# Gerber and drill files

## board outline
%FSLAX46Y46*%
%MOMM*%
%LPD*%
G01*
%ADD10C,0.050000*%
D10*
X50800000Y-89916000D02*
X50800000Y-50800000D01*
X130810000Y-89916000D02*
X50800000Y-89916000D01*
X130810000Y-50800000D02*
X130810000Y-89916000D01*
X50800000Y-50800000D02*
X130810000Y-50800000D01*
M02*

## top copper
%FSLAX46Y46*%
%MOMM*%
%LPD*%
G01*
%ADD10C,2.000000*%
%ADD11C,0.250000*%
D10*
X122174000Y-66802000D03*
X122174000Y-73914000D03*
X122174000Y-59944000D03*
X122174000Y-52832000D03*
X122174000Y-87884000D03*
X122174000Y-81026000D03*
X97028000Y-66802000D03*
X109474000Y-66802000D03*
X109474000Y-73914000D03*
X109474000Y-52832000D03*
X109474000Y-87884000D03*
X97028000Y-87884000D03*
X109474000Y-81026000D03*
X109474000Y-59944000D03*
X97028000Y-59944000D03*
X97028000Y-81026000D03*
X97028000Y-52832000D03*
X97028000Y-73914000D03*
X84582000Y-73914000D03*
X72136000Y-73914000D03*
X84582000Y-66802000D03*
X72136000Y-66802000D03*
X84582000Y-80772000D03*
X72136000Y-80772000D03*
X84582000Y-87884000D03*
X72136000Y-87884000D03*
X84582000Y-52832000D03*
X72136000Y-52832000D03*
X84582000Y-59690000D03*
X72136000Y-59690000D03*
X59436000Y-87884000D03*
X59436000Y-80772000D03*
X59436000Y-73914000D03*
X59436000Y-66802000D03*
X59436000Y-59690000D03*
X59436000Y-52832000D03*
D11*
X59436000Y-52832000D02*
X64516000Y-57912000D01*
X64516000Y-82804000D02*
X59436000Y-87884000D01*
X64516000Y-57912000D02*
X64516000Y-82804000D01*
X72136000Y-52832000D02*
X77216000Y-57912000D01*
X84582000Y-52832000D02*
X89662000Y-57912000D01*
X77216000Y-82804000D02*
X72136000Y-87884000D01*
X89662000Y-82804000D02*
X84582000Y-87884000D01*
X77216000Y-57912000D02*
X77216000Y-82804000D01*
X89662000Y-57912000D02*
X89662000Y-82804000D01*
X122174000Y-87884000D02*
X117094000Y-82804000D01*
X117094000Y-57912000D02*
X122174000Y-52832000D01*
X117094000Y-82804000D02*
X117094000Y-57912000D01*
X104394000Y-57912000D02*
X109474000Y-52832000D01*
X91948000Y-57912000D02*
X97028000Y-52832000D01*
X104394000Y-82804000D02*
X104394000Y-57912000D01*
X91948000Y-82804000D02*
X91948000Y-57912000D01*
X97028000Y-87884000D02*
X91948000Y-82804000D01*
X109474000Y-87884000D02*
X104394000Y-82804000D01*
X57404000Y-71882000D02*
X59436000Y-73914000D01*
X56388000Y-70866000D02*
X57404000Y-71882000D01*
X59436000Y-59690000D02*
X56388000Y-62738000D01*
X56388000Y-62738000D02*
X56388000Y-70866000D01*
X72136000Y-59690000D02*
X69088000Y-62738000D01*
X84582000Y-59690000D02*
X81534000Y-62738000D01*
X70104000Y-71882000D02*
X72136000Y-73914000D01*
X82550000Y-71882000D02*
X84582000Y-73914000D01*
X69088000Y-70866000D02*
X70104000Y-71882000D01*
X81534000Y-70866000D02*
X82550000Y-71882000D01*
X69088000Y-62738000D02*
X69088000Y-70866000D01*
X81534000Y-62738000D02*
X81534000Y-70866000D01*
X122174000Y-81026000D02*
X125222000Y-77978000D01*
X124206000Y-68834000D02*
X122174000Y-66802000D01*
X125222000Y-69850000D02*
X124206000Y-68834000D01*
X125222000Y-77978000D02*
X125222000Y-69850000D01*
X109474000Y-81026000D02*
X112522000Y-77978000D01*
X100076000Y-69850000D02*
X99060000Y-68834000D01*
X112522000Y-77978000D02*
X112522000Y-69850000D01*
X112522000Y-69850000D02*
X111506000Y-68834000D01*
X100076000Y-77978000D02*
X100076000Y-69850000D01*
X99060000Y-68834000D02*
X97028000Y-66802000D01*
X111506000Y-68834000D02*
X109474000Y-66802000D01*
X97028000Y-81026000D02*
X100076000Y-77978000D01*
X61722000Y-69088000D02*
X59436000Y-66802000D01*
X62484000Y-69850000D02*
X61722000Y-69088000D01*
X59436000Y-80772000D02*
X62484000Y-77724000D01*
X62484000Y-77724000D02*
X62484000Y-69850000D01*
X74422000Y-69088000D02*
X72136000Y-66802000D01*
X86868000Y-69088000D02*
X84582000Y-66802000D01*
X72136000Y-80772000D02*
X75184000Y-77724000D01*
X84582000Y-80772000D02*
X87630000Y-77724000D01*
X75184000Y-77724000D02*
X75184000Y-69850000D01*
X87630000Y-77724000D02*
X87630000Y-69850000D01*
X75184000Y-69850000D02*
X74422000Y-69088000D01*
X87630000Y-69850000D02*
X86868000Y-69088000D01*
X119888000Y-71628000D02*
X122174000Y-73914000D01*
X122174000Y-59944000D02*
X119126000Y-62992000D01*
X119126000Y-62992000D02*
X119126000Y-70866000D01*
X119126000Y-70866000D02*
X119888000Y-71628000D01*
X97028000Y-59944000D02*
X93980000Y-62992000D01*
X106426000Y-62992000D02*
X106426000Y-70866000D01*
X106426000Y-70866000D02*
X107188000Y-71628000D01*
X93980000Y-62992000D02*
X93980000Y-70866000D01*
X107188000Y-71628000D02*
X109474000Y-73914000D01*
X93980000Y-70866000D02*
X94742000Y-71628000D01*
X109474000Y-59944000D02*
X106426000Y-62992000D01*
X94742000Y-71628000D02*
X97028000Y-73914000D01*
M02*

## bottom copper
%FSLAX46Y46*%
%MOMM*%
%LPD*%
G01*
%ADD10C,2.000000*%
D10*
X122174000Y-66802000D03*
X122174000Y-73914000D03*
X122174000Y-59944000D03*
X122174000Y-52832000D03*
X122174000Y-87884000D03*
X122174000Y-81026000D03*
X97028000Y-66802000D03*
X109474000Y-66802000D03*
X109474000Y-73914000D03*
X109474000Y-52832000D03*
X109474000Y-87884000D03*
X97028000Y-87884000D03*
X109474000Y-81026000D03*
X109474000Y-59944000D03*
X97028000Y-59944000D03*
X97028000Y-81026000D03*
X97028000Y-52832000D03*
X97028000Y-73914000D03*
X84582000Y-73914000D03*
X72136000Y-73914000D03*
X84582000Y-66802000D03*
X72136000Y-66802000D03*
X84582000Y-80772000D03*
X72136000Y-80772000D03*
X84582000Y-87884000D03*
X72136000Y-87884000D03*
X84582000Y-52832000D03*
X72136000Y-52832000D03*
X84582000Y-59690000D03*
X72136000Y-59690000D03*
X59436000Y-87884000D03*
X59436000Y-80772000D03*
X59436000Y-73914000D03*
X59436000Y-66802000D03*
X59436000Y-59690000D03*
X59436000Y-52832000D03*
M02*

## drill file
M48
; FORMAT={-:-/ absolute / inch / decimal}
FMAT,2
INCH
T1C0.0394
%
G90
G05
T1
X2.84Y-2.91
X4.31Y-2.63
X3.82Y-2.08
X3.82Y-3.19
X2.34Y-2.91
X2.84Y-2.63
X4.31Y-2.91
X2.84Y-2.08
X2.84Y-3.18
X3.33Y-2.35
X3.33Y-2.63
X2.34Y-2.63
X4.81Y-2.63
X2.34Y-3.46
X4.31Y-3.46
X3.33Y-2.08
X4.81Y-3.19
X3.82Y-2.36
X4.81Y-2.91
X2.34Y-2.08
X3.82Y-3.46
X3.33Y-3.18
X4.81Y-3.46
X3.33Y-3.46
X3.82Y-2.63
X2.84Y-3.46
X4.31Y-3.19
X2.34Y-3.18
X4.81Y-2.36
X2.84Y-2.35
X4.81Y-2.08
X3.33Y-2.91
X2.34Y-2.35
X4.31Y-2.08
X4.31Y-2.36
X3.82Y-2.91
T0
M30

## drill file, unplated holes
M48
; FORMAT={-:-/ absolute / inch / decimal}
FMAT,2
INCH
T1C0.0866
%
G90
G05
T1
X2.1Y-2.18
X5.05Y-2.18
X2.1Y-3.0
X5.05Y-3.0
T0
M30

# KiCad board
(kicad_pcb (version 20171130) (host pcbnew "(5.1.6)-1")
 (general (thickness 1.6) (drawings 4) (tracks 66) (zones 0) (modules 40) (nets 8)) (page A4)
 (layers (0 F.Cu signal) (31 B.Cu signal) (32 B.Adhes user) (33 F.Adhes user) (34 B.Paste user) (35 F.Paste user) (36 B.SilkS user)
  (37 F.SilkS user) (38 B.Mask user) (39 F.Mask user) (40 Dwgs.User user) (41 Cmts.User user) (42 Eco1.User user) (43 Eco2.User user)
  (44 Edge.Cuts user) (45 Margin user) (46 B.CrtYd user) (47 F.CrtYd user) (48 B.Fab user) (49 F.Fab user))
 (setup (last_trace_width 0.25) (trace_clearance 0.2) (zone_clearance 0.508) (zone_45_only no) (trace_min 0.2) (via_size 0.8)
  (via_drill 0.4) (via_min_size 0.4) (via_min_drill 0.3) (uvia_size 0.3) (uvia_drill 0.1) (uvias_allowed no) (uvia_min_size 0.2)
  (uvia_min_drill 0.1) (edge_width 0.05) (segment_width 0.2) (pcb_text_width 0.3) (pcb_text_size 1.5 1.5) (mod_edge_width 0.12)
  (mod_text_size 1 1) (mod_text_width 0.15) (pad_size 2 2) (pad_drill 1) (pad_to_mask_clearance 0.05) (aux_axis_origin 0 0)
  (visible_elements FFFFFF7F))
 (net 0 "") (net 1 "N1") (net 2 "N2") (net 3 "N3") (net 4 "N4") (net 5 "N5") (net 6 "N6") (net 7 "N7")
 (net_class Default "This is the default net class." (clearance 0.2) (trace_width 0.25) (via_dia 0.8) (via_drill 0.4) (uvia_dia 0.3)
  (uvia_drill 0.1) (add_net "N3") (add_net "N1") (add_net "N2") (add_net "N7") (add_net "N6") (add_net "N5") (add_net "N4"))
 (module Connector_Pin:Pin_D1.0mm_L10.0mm (layer F.Cu) (at 122.174 66.802 180)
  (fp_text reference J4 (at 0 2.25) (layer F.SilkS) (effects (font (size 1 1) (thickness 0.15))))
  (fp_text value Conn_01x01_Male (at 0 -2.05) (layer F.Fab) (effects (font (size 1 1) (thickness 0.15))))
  (pad 1 thru_hole circle (at 0 0 180) (size 2 2) (drill 1) (layers *.Cu *.Mask) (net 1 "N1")))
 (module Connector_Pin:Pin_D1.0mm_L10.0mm (layer F.Cu) (at 122.174 73.914 180)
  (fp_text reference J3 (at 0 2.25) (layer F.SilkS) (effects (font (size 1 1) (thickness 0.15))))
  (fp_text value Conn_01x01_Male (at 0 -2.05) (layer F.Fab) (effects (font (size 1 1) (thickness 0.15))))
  (pad 1 thru_hole circle (at 0 0 180) (size 2 2) (drill 1) (layers *.Cu *.Mask) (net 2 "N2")))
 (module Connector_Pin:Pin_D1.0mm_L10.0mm (layer F.Cu) (at 122.174 59.944 180)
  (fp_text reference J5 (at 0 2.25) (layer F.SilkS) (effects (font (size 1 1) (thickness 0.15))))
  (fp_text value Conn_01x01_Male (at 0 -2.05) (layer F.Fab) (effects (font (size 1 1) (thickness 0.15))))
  (pad 1 thru_hole circle (at 0 0 180) (size 2 2) (drill 1) (layers *.Cu *.Mask) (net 2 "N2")))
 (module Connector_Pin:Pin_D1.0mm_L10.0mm (layer F.Cu) (at 122.174 52.832 180)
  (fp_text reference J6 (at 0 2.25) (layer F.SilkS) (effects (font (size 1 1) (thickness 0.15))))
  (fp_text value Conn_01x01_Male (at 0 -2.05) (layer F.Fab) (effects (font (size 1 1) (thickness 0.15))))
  (pad 1 thru_hole circle (at 0 0 180) (size 2 2) (drill 1) (layers *.Cu *.Mask) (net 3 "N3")))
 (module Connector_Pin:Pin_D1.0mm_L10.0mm (layer F.Cu) (at 122.174 87.884 180)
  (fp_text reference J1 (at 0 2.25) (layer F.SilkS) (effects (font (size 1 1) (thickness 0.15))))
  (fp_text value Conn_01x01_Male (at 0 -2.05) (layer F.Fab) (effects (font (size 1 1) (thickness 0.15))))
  (pad 1 thru_hole circle (at 0 0 180) (size 2 2) (drill 1) (layers *.Cu *.Mask) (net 3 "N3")))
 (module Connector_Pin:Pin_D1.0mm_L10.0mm (layer F.Cu) (at 122.174 81.026 180)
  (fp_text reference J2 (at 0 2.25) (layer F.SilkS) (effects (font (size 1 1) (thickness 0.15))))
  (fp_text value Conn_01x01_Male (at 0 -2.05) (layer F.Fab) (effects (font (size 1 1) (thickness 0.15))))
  (pad 1 thru_hole circle (at 0 0 180) (size 2 2) (drill 1) (layers *.Cu *.Mask) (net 1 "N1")))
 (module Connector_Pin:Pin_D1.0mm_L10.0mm (layer F.Cu) (at 97.028 66.802 180)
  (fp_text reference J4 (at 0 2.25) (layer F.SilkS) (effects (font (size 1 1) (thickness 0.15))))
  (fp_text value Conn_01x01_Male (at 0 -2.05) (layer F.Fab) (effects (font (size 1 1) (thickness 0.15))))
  (pad 1 thru_hole circle (at 0 0 180) (size 2 2) (drill 1) (layers *.Cu *.Mask) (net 1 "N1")))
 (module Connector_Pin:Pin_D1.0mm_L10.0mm (layer F.Cu) (at 109.474 66.802 180)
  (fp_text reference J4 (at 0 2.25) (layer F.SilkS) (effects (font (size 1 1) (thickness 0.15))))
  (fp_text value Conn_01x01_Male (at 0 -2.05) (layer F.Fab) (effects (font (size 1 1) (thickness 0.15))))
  (pad 1 thru_hole circle (at 0 0 180) (size 2 2) (drill 1) (layers *.Cu *.Mask) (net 1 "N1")))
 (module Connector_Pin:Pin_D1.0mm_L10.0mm (layer F.Cu) (at 109.474 73.914 180)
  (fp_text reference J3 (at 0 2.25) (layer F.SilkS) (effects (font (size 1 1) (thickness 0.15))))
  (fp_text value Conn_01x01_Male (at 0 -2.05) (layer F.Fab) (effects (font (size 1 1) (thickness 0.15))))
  (pad 1 thru_hole circle (at 0 0 180) (size 2 2) (drill 1) (layers *.Cu *.Mask) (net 2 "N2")))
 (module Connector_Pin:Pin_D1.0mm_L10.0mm (layer F.Cu) (at 109.474 52.832 180)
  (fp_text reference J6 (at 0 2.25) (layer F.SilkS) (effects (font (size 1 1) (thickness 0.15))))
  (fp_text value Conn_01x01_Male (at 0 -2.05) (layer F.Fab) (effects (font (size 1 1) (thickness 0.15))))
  (pad 1 thru_hole circle (at 0 0 180) (size 2 2) (drill 1) (layers *.Cu *.Mask) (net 3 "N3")))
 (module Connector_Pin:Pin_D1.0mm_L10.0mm (layer F.Cu) (at 109.474 87.884 180)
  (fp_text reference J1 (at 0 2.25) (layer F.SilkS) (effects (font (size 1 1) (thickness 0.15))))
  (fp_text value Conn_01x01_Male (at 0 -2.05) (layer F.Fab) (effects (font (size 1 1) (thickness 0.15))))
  (pad 1 thru_hole circle (at 0 0 180) (size 2 2) (drill 1) (layers *.Cu *.Mask) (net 3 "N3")))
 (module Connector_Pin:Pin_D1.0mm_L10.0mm (layer F.Cu) (at 97.028 87.884 180)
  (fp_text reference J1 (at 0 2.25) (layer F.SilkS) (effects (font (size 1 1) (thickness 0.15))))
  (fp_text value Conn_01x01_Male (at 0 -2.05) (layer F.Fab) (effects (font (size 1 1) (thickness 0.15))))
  (pad 1 thru_hole circle (at 0 0 180) (size 2 2) (drill 1) (layers *.Cu *.Mask) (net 3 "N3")))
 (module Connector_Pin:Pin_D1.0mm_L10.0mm (layer F.Cu) (at 109.474 81.026 180)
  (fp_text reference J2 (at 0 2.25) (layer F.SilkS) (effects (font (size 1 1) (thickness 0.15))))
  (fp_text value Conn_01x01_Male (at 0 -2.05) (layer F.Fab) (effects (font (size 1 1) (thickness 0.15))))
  (pad 1 thru_hole circle (at 0 0 180) (size 2 2) (drill 1) (layers *.Cu *.Mask) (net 1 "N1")))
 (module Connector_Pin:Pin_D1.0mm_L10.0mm (layer F.Cu) (at 109.474 59.944 180)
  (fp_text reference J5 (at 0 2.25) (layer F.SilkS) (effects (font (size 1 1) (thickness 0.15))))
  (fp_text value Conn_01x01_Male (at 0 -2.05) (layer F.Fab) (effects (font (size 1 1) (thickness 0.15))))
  (pad 1 thru_hole circle (at 0 0 180) (size 2 2) (drill 1) (layers *.Cu *.Mask) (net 2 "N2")))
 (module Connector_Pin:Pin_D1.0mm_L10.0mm (layer F.Cu) (at 97.028 59.944 180)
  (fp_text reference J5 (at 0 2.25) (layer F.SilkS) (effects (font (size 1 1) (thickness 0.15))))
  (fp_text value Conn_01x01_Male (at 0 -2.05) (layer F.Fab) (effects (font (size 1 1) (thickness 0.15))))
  (pad 1 thru_hole circle (at 0 0 180) (size 2 2) (drill 1) (layers *.Cu *.Mask) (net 2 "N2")))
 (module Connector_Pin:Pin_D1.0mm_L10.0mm (layer F.Cu) (at 97.028 81.026 180)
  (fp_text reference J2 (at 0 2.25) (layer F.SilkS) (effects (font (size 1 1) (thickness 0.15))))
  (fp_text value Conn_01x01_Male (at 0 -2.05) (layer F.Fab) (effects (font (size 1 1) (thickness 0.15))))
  (pad 1 thru_hole circle (at 0 0 180) (size 2 2) (drill 1) (layers *.Cu *.Mask) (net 1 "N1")))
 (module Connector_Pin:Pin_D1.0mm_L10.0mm (layer F.Cu) (at 97.028 52.832 180)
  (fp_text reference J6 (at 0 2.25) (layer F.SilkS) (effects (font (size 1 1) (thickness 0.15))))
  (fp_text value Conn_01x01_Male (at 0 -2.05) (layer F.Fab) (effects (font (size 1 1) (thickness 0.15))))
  (pad 1 thru_hole circle (at 0 0 180) (size 2 2) (drill 1) (layers *.Cu *.Mask) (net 3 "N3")))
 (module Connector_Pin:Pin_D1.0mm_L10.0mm (layer F.Cu) (at 97.028 73.914 180)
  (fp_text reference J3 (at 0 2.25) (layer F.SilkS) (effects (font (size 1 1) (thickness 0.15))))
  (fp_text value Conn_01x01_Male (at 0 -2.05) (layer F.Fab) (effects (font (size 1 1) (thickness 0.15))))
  (pad 1 thru_hole circle (at 0 0 180) (size 2 2) (drill 1) (layers *.Cu *.Mask) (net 2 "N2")))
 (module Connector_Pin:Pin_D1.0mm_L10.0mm (layer F.Cu) (at 84.582 73.914)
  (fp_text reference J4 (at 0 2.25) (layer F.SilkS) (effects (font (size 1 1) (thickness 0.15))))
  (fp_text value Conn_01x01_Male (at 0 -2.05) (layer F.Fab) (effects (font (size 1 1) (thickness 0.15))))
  (pad 1 thru_hole circle (at 0 0) (size 2 2) (drill 1) (layers *.Cu *.Mask) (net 1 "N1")))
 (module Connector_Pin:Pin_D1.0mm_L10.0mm (layer F.Cu) (at 72.136 73.914)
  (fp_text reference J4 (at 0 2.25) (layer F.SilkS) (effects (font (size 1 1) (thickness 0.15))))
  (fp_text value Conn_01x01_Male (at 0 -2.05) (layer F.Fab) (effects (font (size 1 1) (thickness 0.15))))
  (pad 1 thru_hole circle (at 0 0) (size 2 2) (drill 1) (layers *.Cu *.Mask) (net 1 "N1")))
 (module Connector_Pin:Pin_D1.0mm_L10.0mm (layer F.Cu) (at 84.582 66.802)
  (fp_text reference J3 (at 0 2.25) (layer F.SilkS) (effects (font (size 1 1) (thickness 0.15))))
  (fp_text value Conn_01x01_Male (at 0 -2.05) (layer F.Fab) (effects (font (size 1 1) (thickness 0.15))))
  (pad 1 thru_hole circle (at 0 0) (size 2 2) (drill 1) (layers *.Cu *.Mask) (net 2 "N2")))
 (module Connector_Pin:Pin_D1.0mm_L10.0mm (layer F.Cu) (at 72.136 66.802)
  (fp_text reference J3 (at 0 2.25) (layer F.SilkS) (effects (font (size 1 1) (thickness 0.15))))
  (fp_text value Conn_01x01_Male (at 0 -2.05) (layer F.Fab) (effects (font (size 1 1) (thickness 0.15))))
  (pad 1 thru_hole circle (at 0 0) (size 2 2) (drill 1) (layers *.Cu *.Mask) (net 2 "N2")))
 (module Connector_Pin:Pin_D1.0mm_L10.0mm (layer F.Cu) (at 84.582 80.772)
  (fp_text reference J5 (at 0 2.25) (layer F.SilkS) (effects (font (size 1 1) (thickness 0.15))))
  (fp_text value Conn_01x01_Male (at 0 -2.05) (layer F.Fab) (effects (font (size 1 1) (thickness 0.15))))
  (pad 1 thru_hole circle (at 0 0) (size 2 2) (drill 1) (layers *.Cu *.Mask) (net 2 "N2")))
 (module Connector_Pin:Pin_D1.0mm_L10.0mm (layer F.Cu) (at 72.136 80.772)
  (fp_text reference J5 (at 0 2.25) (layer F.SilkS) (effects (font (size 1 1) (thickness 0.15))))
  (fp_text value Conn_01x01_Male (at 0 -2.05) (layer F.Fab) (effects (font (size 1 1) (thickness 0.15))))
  (pad 1 thru_hole circle (at 0 0) (size 2 2) (drill 1) (layers *.Cu *.Mask) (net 2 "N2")))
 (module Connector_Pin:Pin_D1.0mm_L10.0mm (layer F.Cu) (at 84.582 87.884)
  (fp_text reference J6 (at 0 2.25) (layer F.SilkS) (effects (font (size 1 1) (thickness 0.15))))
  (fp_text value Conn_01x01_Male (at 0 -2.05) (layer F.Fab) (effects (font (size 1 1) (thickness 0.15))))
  (pad 1 thru_hole circle (at 0 0) (size 2 2) (drill 1) (layers *.Cu *.Mask) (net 3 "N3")))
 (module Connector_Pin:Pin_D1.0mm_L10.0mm (layer F.Cu) (at 72.136 87.884)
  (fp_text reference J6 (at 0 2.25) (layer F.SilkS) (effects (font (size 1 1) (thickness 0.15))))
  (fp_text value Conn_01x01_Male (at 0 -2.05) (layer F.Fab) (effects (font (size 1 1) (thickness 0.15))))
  (pad 1 thru_hole circle (at 0 0) (size 2 2) (drill 1) (layers *.Cu *.Mask) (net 3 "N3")))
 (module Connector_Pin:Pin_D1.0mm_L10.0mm (layer F.Cu) (at 84.582 52.832)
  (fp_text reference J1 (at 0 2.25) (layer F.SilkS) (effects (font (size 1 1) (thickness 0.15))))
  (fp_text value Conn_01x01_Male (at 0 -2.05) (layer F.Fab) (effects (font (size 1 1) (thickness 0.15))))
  (pad 1 thru_hole circle (at 0 0) (size 2 2) (drill 1) (layers *.Cu *.Mask) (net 3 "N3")))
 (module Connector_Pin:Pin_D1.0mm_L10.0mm (layer F.Cu) (at 72.136 52.832)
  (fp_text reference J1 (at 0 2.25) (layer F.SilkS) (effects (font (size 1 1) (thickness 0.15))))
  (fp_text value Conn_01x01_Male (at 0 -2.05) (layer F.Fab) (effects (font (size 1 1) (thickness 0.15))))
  (pad 1 thru_hole circle (at 0 0) (size 2 2) (drill 1) (layers *.Cu *.Mask) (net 3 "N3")))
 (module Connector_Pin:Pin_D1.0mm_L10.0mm (layer F.Cu) (at 84.582 59.69)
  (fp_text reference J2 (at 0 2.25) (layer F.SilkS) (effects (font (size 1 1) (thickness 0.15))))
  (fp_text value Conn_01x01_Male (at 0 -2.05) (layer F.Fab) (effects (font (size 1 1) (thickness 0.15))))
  (pad 1 thru_hole circle (at 0 0) (size 2 2) (drill 1) (layers *.Cu *.Mask) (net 1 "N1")))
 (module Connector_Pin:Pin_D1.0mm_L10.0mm (layer F.Cu) (at 72.136 59.69)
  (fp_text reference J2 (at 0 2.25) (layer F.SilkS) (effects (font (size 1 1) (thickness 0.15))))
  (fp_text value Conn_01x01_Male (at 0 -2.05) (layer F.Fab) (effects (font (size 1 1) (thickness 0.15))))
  (pad 1 thru_hole circle (at 0 0) (size 2 2) (drill 1) (layers *.Cu *.Mask) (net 1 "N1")))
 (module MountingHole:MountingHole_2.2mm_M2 (layer F.Cu) (at 53.34 76.2)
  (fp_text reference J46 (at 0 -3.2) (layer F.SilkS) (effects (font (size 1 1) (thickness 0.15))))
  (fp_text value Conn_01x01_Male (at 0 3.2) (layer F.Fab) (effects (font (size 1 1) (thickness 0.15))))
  (pad 1 np_thru_hole circle (at 0 0) (size 2.2 2.2) (drill 2.2) (layers *.Cu *.Mask) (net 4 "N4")))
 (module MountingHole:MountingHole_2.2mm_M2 (layer F.Cu) (at 128.27 76.2)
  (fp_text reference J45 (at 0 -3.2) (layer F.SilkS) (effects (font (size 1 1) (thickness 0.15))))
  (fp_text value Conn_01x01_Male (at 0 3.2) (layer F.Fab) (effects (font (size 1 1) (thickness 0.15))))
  (pad 1 np_thru_hole circle (at 0 0) (size 2.2 2.2) (drill 2.2) (layers *.Cu *.Mask) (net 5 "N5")))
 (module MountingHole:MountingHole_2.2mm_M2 (layer F.Cu) (at 128.27 55.372)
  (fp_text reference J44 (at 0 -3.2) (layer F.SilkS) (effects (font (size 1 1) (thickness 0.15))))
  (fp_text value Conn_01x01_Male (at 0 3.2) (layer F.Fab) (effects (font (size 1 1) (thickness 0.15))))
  (pad 1 np_thru_hole circle (at 0 0) (size 2.2 2.2) (drill 2.2) (layers *.Cu *.Mask) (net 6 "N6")))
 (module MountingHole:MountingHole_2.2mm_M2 (layer F.Cu) (at 53.34 55.372)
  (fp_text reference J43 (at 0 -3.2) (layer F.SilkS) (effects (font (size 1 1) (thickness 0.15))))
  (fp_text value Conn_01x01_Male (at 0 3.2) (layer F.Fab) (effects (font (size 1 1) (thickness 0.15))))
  (pad 1 np_thru_hole circle (at 0 0) (size 2.2 2.2) (drill 2.2) (layers *.Cu *.Mask) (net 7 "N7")))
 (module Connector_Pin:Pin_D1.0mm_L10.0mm (layer F.Cu) (at 59.436 87.884)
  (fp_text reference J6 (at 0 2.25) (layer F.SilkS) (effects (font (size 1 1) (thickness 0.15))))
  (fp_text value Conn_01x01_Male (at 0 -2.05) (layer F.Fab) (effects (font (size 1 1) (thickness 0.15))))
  (pad 1 thru_hole circle (at 0 0) (size 2 2) (drill 1) (layers *.Cu *.Mask) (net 3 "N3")))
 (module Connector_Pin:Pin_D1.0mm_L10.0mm (layer F.Cu) (at 59.436 80.772)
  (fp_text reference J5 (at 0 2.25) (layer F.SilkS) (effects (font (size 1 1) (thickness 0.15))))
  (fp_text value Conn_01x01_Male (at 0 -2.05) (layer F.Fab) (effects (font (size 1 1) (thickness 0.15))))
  (pad 1 thru_hole circle (at 0 0) (size 2 2) (drill 1) (layers *.Cu *.Mask) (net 2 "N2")))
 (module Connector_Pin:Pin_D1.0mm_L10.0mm (layer F.Cu) (at 59.436 73.914)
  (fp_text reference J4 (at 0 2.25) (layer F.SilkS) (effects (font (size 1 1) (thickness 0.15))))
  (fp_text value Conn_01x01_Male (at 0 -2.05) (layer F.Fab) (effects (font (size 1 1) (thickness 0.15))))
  (pad 1 thru_hole circle (at 0 0) (size 2 2) (drill 1) (layers *.Cu *.Mask) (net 1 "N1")))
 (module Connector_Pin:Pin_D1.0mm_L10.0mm (layer F.Cu) (at 59.436 66.802)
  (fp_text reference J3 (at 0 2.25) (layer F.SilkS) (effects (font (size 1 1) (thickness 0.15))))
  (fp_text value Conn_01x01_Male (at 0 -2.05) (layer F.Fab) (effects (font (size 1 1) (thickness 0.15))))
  (pad 1 thru_hole circle (at 0 0) (size 2 2) (drill 1) (layers *.Cu *.Mask) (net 2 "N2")))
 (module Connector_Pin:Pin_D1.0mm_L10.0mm (layer F.Cu) (at 59.436 59.69)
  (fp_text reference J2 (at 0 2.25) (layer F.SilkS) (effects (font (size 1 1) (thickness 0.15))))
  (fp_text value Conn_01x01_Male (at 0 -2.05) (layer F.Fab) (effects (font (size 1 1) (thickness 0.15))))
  (pad 1 thru_hole circle (at 0 0) (size 2 2) (drill 1) (layers *.Cu *.Mask) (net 1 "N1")))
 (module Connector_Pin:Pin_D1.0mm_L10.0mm (layer F.Cu) (at 59.436 52.832)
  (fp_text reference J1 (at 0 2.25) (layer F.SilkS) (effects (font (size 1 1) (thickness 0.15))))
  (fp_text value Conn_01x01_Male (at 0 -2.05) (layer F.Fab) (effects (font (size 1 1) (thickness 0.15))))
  (pad 1 thru_hole circle (at 0 0) (size 2 2) (drill 1) (layers *.Cu *.Mask) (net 3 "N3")))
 (gr_line (start 50.8 89.916) (end 50.8 50.8) (layer Edge.Cuts) (width 0.05))
 (gr_line (start 130.81 89.916) (end 50.8 89.916) (layer Edge.Cuts) (width 0.05))
 (gr_line (start 130.81 50.8) (end 130.81 89.916) (layer Edge.Cuts) (width 0.05))
 (gr_line (start 50.8 50.8) (end 130.81 50.8) (layer Edge.Cuts) (width 0.05))
 (segment (start 59.436 52.832) (end 64.516 57.912) (width 0.25) (layer F.Cu) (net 3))
 (segment (start 64.516 82.804) (end 59.436 87.884) (width 0.25) (layer F.Cu) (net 3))
 (segment (start 64.516 57.912) (end 64.516 82.804) (width 0.25) (layer F.Cu) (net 3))
 (segment (start 72.136 52.832) (end 77.216 57.912) (width 0.25) (layer F.Cu) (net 3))
 (segment (start 84.582 52.832) (end 89.662 57.912) (width 0.25) (layer F.Cu) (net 3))
 (segment (start 77.216 82.804) (end 72.136 87.884) (width 0.25) (layer F.Cu) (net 3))
 (segment (start 89.662 82.804) (end 84.582 87.884) (width 0.25) (layer F.Cu) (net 3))
 (segment (start 77.216 57.912) (end 77.216 82.804) (width 0.25) (layer F.Cu) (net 3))
 (segment (start 89.662 57.912) (end 89.662 82.804) (width 0.25) (layer F.Cu) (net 3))
 (segment (start 122.174 87.884) (end 117.094 82.804) (width 0.25) (layer F.Cu) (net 3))
 (segment (start 117.094 57.912) (end 122.174 52.832) (width 0.25) (layer F.Cu) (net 3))
 (segment (start 117.094 82.804) (end 117.094 57.912) (width 0.25) (layer F.Cu) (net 3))
 (segment (start 104.394 57.912) (end 109.474 52.832) (width 0.25) (layer F.Cu) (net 3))
 (segment (start 91.948 57.912) (end 97.028 52.832) (width 0.25) (layer F.Cu) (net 3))
 (segment (start 104.394 82.804) (end 104.394 57.912) (width 0.25) (layer F.Cu) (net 3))
 (segment (start 91.948 82.804) (end 91.948 57.912) (width 0.25) (layer F.Cu) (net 3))
 (segment (start 97.028 87.884) (end 91.948 82.804) (width 0.25) (layer F.Cu) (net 3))
 (segment (start 109.474 87.884) (end 104.394 82.804) (width 0.25) (layer F.Cu) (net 3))
 (segment (start 57.404 71.882) (end 59.436 73.914) (width 0.25) (layer F.Cu) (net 1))
 (segment (start 56.388 70.866) (end 57.404 71.882) (width 0.25) (layer F.Cu) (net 1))
 (segment (start 59.436 59.69) (end 56.388 62.738) (width 0.25) (layer F.Cu) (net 1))
 (segment (start 56.388 62.738) (end 56.388 70.866) (width 0.25) (layer F.Cu) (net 1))
 (segment (start 72.136 59.69) (end 69.088 62.738) (width 0.25) (layer F.Cu) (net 1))
 (segment (start 84.582 59.69) (end 81.534 62.738) (width 0.25) (layer F.Cu) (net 1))
 (segment (start 70.104 71.882) (end 72.136 73.914) (width 0.25) (layer F.Cu) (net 1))
 (segment (start 82.55 71.882) (end 84.582 73.914) (width 0.25) (layer F.Cu) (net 1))
 (segment (start 69.088 70.866) (end 70.104 71.882) (width 0.25) (layer F.Cu) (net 1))
 (segment (start 81.534 70.866) (end 82.55 71.882) (width 0.25) (layer F.Cu) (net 1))
 (segment (start 69.088 62.738) (end 69.088 70.866) (width 0.25) (layer F.Cu) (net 1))
 (segment (start 81.534 62.738) (end 81.534 70.866) (width 0.25) (layer F.Cu) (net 1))
 (segment (start 122.174 81.026) (end 125.222 77.978) (width 0.25) (layer F.Cu) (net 1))
 (segment (start 124.206 68.834) (end 122.174 66.802) (width 0.25) (layer F.Cu) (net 1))
 (segment (start 125.222 69.85) (end 124.206 68.834) (width 0.25) (layer F.Cu) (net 1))
 (segment (start 125.222 77.978) (end 125.222 69.85) (width 0.25) (layer F.Cu) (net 1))
 (segment (start 109.474 81.026) (end 112.522 77.978) (width 0.25) (layer F.Cu) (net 1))
 (segment (start 100.076 69.85) (end 99.06 68.834) (width 0.25) (layer F.Cu) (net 1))
 (segment (start 112.522 77.978) (end 112.522 69.85) (width 0.25) (layer F.Cu) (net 1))
 (segment (start 112.522 69.85) (end 111.506 68.834) (width 0.25) (layer F.Cu) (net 1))
 (segment (start 100.076 77.978) (end 100.076 69.85) (width 0.25) (layer F.Cu) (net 1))
 (segment (start 99.06 68.834) (end 97.028 66.802) (width 0.25) (layer F.Cu) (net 1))
 (segment (start 111.506 68.834) (end 109.474 66.802) (width 0.25) (layer F.Cu) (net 1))
 (segment (start 97.028 81.026) (end 100.076 77.978) (width 0.25) (layer F.Cu) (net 1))
 (segment (start 61.722 69.088) (end 59.436 66.802) (width 0.25) (layer F.Cu) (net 2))
 (segment (start 62.484 69.85) (end 61.722 69.088) (width 0.25) (layer F.Cu) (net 2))
 (segment (start 59.436 80.772) (end 62.484 77.724) (width 0.25) (layer F.Cu) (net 2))
 (segment (start 62.484 77.724) (end 62.484 69.85) (width 0.25) (layer F.Cu) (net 2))
 (segment (start 74.422 69.088) (end 72.136 66.802) (width 0.25) (layer F.Cu) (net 2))
 (segment (start 86.868 69.088) (end 84.582 66.802) (width 0.25) (layer F.Cu) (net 2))
 (segment (start 72.136 80.772) (end 75.184 77.724) (width 0.25) (layer F.Cu) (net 2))
 (segment (start 84.582 80.772) (end 87.63 77.724) (width 0.25) (layer F.Cu) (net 2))
 (segment (start 75.184 77.724) (end 75.184 69.85) (width 0.25) (layer F.Cu) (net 2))
 (segment (start 87.63 77.724) (end 87.63 69.85) (width 0.25) (layer F.Cu) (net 2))
 (segment (start 75.184 69.85) (end 74.422 69.088) (width 0.25) (layer F.Cu) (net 2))
 (segment (start 87.63 69.85) (end 86.868 69.088) (width 0.25) (layer F.Cu) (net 2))
 (segment (start 119.888 71.628) (end 122.174 73.914) (width 0.25) (layer F.Cu) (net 2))
 (segment (start 122.174 59.944) (end 119.126 62.992) (width 0.25) (layer F.Cu) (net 2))
 (segment (start 119.126 62.992) (end 119.126 70.866) (width 0.25) (layer F.Cu) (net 2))
 (segment (start 119.126 70.866) (end 119.888 71.628) (width 0.25) (layer F.Cu) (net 2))
 (segment (start 97.028 59.944) (end 93.98 62.992) (width 0.25) (layer F.Cu) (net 2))
 (segment (start 106.426 62.992) (end 106.426 70.866) (width 0.25) (layer F.Cu) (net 2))
 (segment (start 106.426 70.866) (end 107.188 71.628) (width 0.25) (layer F.Cu) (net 2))
 (segment (start 93.98 62.992) (end 93.98 70.866) (width 0.25) (layer F.Cu) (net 2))
 (segment (start 107.188 71.628) (end 109.474 73.914) (width 0.25) (layer F.Cu) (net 2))
 (segment (start 93.98 70.866) (end 94.742 71.628) (width 0.25) (layer F.Cu) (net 2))
 (segment (start 109.474 59.944) (end 106.426 62.992) (width 0.25) (layer F.Cu) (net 2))
 (segment (start 94.742 71.628) (end 97.028 73.914) (width 0.25) (layer F.Cu) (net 2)))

